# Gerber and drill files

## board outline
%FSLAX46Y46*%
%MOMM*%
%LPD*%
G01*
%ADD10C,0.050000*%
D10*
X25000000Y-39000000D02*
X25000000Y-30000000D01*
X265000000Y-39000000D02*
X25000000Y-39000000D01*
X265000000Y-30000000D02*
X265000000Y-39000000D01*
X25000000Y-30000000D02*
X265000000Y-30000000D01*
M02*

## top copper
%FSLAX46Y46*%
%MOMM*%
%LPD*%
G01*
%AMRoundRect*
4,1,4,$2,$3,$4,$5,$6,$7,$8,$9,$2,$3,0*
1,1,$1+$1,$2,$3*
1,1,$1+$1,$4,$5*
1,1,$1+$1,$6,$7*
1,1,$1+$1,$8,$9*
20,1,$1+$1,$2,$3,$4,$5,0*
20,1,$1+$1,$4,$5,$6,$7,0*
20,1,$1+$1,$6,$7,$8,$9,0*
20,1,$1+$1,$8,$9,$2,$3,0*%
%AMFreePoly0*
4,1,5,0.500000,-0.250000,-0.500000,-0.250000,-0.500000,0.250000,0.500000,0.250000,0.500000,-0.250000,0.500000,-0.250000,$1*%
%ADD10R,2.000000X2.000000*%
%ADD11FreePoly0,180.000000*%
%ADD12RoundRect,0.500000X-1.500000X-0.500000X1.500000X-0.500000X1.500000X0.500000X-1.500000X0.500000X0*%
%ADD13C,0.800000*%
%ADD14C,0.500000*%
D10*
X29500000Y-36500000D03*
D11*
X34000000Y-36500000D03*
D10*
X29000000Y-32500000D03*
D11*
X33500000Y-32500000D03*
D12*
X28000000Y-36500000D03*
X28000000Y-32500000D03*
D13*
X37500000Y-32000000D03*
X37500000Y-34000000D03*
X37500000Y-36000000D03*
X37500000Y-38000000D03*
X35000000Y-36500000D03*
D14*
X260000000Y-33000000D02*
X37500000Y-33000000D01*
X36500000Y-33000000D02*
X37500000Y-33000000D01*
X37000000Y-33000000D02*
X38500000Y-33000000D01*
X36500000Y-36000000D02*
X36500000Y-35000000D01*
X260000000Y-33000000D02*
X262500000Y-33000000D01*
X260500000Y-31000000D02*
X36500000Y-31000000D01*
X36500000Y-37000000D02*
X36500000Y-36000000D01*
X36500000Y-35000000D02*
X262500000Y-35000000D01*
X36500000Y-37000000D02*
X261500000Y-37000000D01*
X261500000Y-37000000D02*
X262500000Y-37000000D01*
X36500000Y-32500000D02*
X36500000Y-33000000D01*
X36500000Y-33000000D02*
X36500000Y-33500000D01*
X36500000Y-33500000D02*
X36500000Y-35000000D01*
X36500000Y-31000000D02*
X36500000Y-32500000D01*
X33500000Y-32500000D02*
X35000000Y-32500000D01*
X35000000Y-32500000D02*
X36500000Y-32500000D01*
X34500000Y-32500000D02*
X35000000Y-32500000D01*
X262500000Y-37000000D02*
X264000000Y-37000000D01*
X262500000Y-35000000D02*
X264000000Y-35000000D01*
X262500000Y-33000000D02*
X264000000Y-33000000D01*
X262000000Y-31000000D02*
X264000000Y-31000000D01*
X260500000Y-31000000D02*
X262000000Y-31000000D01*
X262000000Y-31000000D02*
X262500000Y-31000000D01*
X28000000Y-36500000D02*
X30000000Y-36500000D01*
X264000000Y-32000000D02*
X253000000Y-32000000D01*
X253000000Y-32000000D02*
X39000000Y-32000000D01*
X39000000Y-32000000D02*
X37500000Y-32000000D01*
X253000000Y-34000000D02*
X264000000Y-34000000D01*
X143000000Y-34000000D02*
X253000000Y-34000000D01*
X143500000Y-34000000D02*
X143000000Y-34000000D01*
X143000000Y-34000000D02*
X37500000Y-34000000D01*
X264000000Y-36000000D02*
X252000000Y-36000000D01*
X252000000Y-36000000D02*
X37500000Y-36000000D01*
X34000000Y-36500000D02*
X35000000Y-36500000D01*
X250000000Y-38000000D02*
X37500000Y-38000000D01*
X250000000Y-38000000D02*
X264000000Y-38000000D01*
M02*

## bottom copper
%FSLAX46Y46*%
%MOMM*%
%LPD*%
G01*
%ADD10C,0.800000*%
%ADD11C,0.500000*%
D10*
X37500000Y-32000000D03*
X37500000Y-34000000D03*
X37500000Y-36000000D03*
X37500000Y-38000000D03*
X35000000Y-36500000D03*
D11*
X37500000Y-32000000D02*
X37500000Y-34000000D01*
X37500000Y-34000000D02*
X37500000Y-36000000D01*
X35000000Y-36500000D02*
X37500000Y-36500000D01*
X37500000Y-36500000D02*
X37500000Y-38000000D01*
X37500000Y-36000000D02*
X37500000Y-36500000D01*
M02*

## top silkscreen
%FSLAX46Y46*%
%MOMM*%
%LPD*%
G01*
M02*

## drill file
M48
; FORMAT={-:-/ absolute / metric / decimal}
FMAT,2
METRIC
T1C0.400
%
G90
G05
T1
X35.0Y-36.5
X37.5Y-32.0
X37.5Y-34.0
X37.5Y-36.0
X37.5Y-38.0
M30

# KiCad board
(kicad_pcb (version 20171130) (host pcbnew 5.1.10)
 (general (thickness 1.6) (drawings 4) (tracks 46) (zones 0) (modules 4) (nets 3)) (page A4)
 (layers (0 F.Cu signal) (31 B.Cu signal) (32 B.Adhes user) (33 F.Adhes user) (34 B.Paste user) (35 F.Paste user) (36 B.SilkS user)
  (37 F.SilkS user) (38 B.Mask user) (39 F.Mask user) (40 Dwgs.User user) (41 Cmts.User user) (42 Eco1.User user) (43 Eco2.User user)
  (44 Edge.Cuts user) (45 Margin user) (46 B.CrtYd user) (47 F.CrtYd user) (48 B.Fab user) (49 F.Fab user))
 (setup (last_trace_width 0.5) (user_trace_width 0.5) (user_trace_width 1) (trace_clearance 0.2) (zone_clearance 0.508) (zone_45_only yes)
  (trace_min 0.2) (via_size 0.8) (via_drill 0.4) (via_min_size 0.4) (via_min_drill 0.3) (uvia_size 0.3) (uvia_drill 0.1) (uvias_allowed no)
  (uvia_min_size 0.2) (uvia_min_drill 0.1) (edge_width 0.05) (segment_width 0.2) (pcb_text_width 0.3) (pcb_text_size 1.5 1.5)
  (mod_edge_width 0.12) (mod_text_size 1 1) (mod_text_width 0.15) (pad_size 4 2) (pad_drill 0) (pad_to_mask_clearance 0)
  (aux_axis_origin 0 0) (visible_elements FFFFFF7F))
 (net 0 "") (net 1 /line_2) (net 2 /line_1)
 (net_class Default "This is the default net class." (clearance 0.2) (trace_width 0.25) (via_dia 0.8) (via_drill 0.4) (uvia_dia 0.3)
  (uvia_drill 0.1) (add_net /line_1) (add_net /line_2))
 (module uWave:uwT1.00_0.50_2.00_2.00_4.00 (layer F.Cu) (at 34 36.5 180)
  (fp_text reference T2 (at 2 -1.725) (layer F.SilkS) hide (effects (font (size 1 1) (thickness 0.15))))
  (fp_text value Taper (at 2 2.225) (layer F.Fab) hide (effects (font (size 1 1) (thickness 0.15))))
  (pad 1 smd rect (at 4.5 0 180) (size 2 2) (layers F.Cu) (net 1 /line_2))
  (pad 1 smd custom (at 0 0 180) (size 1 0.5) (layers F.Cu) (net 1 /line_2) (options (clearance outline) (anchor rect)) (primitives)))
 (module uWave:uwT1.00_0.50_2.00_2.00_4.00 (layer F.Cu) (at 33.5 32.5 180)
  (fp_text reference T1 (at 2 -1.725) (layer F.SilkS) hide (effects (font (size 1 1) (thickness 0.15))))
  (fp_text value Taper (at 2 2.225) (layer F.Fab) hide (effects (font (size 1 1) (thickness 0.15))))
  (pad 1 smd rect (at 4.5 0 180) (size 2 2) (layers F.Cu) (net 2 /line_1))
  (pad 1 smd custom (at 0 0 180) (size 1 0.5) (layers F.Cu) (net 2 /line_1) (options (clearance outline) (anchor rect)) (primitives)))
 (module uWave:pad (layer F.Cu) (at 28 37)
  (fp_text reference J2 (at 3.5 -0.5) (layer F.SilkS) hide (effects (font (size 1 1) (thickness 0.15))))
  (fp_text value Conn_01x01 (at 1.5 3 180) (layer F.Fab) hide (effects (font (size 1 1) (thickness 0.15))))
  (pad 1 smd roundrect (at 0 -0.5) (size 4 2) (layers F.Cu F.Paste F.Mask) (roundrect_rratio 0.25) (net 1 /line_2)))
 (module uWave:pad (layer F.Cu) (at 28 33)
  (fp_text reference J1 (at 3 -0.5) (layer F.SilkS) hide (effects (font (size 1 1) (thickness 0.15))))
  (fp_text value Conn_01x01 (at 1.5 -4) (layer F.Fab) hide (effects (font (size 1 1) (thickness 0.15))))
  (pad 1 smd roundrect (at 0 -0.5) (size 4 2) (layers F.Cu F.Paste F.Mask) (roundrect_rratio 0.25) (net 2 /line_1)))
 (gr_line (start 25 39) (end 25 30) (layer Edge.Cuts) (width 0.05))
 (gr_line (start 265 39) (end 25 39) (layer Edge.Cuts) (width 0.05))
 (gr_line (start 265 30) (end 265 39) (layer Edge.Cuts) (width 0.05))
 (gr_line (start 25 30) (end 265 30) (layer Edge.Cuts) (width 0.05))
 (segment (start 260 33) (end 37.5 33) (width 0.5) (layer F.Cu) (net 2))
 (segment (start 36.5 33) (end 37.5 33) (width 0.5) (layer F.Cu) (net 2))
 (segment (start 37 33) (end 38.5 33) (width 0.5) (layer F.Cu) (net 2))
 (segment (start 36.5 36) (end 36.5 35) (width 0.5) (layer F.Cu) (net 2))
 (segment (start 260 33) (end 262.5 33) (width 0.5) (layer F.Cu) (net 2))
 (segment (start 260.5 31) (end 36.5 31) (width 0.5) (layer F.Cu) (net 2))
 (segment (start 36.5 37) (end 36.5 36) (width 0.5) (layer F.Cu) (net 2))
 (segment (start 36.5 35) (end 262.5 35) (width 0.5) (layer F.Cu) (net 2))
 (segment (start 36.5 37) (end 261.5 37) (width 0.5) (layer F.Cu) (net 2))
 (segment (start 261.5 37) (end 262.5 37) (width 0.5) (layer F.Cu) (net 2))
 (segment (start 36.5 32.5) (end 36.5 33) (width 0.5) (layer F.Cu) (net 2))
 (segment (start 36.5 33) (end 36.5 33.5) (width 0.5) (layer F.Cu) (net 2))
 (segment (start 36.5 33.5) (end 36.5 35) (width 0.5) (layer F.Cu) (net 2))
 (segment (start 36.5 31) (end 36.5 32.5) (width 0.5) (layer F.Cu) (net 2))
 (segment (start 33.5 32.5) (end 35 32.5) (width 0.5) (layer F.Cu) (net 2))
 (segment (start 35 32.5) (end 36.5 32.5) (width 0.5) (layer F.Cu) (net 2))
 (segment (start 34.5 32.5) (end 35 32.5) (width 0.5) (layer F.Cu) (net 2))
 (segment (start 262.5 37) (end 264 37) (width 0.5) (layer F.Cu) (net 2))
 (segment (start 262.5 35) (end 264 35) (width 0.5) (layer F.Cu) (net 2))
 (segment (start 262.5 33) (end 264 33) (width 0.5) (layer F.Cu) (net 2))
 (segment (start 262 31) (end 264 31) (width 0.5) (layer F.Cu) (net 2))
 (segment (start 260.5 31) (end 262 31) (width 0.5) (layer F.Cu) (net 2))
 (segment (start 262 31) (end 262.5 31) (width 0.5) (layer F.Cu) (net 2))
 (segment (start 28 36.5) (end 30 36.5) (width 0.5) (layer F.Cu) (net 1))
 (segment (start 264 32) (end 253 32) (width 0.5) (layer F.Cu) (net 1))
 (segment (start 253 32) (end 39 32) (width 0.5) (layer F.Cu) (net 1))
 (segment (start 39 32) (end 37.5 32) (width 0.5) (layer F.Cu) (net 1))
 (segment (start 253 34) (end 264 34) (width 0.5) (layer F.Cu) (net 1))
 (segment (start 143 34) (end 253 34) (width 0.5) (layer F.Cu) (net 1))
 (segment (start 143.5 34) (end 143 34) (width 0.5) (layer F.Cu) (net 1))
 (segment (start 143 34) (end 37.5 34) (width 0.5) (layer F.Cu) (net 1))
 (segment (start 264 36) (end 252 36) (width 0.5) (layer F.Cu) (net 1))
 (segment (start 252 36) (end 37.5 36) (width 0.5) (layer F.Cu) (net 1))
 (via (at 37.5 32) (size 0.8) (drill 0.4) (layers F.Cu B.Cu) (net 1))
 (segment (start 37.5 32) (end 37.5 34) (width 0.5) (layer B.Cu) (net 1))
 (via (at 37.5 34) (size 0.8) (drill 0.4) (layers F.Cu B.Cu) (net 1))
 (segment (start 37.5 34) (end 37.5 36) (width 0.5) (layer B.Cu) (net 1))
 (via (at 37.5 36) (size 0.8) (drill 0.4) (layers F.Cu B.Cu) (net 1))
 (via (at 37.5 38) (size 0.8) (drill 0.4) (layers F.Cu B.Cu) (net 1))
 (via (at 35 36.5) (size 0.8) (drill 0.4) (layers F.Cu B.Cu) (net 1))
 (segment (start 35 36.5) (end 37.5 36.5) (width 0.5) (layer B.Cu) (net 1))
 (segment (start 37.5 36.5) (end 37.5 38) (width 0.5) (layer B.Cu) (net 1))
 (segment (start 37.5 36) (end 37.5 36.5) (width 0.5) (layer B.Cu) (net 1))
 (segment (start 34 36.5) (end 35 36.5) (width 0.5) (layer F.Cu) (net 1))
 (segment (start 250 38) (end 37.5 38) (width 0.5) (layer F.Cu) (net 1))
 (segment (start 250 38) (end 264 38) (width 0.5) (layer F.Cu) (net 1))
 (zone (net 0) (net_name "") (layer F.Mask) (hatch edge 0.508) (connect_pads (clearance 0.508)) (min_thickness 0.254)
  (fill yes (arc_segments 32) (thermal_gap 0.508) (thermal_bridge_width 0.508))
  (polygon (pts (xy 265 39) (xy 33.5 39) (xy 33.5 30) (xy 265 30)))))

